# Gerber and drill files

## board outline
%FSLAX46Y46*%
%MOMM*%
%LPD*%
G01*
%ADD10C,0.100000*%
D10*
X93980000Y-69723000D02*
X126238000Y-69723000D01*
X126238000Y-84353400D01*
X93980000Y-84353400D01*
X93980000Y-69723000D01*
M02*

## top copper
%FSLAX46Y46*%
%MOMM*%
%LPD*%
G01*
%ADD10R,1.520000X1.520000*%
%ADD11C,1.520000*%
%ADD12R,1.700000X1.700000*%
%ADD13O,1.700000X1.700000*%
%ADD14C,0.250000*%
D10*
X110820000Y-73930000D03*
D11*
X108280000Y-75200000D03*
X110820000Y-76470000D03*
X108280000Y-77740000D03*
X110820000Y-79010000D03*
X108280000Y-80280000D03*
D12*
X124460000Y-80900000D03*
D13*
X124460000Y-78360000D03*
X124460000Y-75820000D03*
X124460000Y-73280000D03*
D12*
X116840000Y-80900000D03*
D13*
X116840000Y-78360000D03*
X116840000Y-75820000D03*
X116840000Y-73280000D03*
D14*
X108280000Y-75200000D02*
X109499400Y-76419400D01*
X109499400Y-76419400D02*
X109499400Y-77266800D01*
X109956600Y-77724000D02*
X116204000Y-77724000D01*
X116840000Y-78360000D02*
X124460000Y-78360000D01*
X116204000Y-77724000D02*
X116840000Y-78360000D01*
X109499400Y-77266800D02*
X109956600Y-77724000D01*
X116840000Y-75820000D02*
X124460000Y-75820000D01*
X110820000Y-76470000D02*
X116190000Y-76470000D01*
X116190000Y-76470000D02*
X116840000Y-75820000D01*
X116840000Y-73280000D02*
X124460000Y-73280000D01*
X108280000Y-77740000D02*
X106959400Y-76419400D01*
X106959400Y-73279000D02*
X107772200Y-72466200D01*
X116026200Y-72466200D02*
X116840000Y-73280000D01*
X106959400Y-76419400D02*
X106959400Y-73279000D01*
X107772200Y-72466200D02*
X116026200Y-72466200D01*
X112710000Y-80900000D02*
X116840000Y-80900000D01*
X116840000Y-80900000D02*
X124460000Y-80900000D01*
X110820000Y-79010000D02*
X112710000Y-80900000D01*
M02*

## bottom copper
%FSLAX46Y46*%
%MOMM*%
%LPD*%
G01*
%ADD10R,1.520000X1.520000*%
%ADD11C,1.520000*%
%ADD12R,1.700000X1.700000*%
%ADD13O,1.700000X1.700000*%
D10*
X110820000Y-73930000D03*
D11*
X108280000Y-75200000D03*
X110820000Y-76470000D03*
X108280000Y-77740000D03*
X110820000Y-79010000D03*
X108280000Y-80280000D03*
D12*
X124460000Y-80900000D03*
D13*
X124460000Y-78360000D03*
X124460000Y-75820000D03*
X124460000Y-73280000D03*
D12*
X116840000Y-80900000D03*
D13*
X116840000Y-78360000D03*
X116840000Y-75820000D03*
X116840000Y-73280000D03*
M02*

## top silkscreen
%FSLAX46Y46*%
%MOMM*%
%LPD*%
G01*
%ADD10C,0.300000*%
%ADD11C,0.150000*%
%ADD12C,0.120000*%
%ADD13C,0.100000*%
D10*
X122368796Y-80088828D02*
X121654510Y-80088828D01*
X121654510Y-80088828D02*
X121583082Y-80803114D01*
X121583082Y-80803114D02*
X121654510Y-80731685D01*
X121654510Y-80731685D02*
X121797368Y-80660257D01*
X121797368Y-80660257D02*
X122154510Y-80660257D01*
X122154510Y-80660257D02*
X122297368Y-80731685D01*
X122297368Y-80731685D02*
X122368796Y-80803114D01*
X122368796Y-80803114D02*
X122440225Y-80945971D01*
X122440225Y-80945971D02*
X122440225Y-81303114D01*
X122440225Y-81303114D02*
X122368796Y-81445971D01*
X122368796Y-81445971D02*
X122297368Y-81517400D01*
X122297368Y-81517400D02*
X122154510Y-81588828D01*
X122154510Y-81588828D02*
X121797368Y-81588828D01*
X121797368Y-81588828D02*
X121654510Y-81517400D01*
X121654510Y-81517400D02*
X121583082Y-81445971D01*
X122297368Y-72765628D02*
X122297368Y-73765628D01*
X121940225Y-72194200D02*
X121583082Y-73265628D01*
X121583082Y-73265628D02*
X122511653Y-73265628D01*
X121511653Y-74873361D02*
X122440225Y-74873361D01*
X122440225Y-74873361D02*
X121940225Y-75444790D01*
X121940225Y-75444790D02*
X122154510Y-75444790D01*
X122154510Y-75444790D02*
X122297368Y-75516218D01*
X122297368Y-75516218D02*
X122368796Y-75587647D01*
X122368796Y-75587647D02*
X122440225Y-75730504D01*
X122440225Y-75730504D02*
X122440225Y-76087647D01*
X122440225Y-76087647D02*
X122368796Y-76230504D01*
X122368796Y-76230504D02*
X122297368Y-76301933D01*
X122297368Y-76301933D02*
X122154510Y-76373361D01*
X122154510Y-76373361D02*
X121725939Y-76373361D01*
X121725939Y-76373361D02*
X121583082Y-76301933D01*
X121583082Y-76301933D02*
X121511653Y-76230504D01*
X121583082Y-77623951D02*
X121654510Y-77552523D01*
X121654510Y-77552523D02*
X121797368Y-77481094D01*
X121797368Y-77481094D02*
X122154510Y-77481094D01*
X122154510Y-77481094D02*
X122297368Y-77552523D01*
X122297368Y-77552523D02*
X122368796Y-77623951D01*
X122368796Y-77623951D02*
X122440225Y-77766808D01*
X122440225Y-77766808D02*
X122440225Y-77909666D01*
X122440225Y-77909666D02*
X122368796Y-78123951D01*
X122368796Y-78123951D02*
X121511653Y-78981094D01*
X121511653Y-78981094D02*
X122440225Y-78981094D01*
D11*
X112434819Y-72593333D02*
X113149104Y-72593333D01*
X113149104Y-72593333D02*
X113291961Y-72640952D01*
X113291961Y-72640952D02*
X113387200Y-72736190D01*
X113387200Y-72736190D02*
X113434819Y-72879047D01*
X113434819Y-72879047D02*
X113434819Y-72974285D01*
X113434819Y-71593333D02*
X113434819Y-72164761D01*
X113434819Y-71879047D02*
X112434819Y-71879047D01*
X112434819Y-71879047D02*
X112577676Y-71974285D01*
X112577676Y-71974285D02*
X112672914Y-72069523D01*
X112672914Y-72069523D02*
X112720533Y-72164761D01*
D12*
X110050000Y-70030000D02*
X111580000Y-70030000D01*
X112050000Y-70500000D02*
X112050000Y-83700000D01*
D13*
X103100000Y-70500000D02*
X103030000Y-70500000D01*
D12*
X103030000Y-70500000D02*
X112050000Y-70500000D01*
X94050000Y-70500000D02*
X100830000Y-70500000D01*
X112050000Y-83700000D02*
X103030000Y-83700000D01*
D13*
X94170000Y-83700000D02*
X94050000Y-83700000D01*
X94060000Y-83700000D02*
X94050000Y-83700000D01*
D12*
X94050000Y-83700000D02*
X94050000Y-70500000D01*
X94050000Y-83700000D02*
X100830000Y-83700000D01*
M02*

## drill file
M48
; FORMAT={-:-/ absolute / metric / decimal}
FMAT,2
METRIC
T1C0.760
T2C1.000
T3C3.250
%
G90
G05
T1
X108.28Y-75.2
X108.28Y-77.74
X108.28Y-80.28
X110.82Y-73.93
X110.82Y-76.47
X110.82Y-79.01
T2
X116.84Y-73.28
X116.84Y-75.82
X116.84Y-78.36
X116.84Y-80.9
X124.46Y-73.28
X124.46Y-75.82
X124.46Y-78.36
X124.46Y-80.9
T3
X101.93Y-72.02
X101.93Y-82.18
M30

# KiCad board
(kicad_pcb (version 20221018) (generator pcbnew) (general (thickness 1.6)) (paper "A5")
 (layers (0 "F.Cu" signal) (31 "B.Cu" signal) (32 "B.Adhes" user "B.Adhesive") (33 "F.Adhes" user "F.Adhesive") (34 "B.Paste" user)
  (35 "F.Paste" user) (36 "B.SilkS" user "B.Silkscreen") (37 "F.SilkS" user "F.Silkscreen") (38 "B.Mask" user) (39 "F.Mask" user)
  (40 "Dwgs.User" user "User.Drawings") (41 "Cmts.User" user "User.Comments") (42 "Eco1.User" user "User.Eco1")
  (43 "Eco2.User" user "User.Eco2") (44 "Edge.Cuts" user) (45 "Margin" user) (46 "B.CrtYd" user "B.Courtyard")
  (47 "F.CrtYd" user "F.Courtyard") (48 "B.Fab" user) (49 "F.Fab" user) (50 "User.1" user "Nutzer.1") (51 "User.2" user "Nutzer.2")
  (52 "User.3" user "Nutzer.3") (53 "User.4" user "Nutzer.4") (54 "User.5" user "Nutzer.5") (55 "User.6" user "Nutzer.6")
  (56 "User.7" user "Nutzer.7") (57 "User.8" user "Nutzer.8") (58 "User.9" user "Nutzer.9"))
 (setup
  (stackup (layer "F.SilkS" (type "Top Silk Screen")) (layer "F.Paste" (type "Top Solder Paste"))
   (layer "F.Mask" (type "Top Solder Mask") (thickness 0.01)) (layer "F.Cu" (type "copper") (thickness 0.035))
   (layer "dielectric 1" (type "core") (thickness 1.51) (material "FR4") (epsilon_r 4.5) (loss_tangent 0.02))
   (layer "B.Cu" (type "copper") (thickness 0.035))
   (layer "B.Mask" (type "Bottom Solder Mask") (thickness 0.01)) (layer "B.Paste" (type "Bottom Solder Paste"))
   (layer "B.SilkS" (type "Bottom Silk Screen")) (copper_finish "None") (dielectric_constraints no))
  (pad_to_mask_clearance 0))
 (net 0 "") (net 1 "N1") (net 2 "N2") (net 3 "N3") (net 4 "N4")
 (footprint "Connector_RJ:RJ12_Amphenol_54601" (layer "F.Cu") (at 110.82 73.93 -90)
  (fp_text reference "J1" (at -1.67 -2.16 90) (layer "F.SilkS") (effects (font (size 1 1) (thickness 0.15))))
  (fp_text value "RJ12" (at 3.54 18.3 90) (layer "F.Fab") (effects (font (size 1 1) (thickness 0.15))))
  (fp_line (start -3.9 0.77) (end -3.9 -0.76) (stroke (width 0.12) (type solid)) (layer "F.SilkS"))
  (fp_line (start -3.43 -1.23) (end 9.77 -1.23) (stroke (width 0.12) (type solid)) (layer "F.SilkS"))
  (fp_line (start -3.43 7.72) (end -3.43 7.79) (stroke (width 0.1) (type solid)) (layer "F.SilkS"))
  (fp_line (start -3.43 7.79) (end -3.43 -1.23) (stroke (width 0.12) (type solid)) (layer "F.SilkS"))
  (fp_line (start -3.43 16.77) (end -3.43 9.99) (stroke (width 0.12) (type solid)) (layer "F.SilkS"))
  (fp_line (start 9.77 -1.23) (end 9.77 7.79) (stroke (width 0.12) (type solid)) (layer "F.SilkS"))
  (fp_line (start 9.77 16.65) (end 9.77 16.77) (stroke (width 0.1) (type solid)) (layer "F.SilkS"))
  (fp_line (start 9.77 16.76) (end 9.77 16.77) (stroke (width 0.1) (type solid)) (layer "F.SilkS"))
  (fp_line (start 9.77 16.77) (end -3.43 16.77) (stroke (width 0.12) (type solid)) (layer "F.SilkS"))
  (fp_line (start 9.77 16.77) (end 9.77 9.99) (stroke (width 0.12) (type solid)) (layer "F.SilkS"))
  (pad "" np_thru_hole circle (at -1.91 8.89 270) (size 3.25 3.25) (drill 3.25) (layers "*.Cu" "*.Mask"))
  (pad "" np_thru_hole circle (at 8.25 8.89 270) (size 3.25 3.25) (drill 3.25) (layers "*.Cu" "*.Mask"))
  (pad "1" thru_hole rect (at 0 0 270) (size 1.52 1.52) (drill 0.76) (layers "*.Cu" "*.Mask"))
  (pad "2" thru_hole circle (at 1.27 2.54 270) (size 1.52 1.52) (drill 0.76) (layers "*.Cu" "*.Mask") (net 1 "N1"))
  (pad "3" thru_hole circle (at 2.54 0 270) (size 1.52 1.52) (drill 0.76) (layers "*.Cu" "*.Mask") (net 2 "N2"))
  (pad "4" thru_hole circle (at 3.81 2.54 270) (size 1.52 1.52) (drill 0.76) (layers "*.Cu" "*.Mask") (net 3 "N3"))
  (pad "5" thru_hole circle (at 5.08 0 270) (size 1.52 1.52) (drill 0.76) (layers "*.Cu" "*.Mask") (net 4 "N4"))
  (pad "6" thru_hole circle (at 6.35 2.54 270) (size 1.52 1.52) (drill 0.76) (layers "*.Cu" "*.Mask")))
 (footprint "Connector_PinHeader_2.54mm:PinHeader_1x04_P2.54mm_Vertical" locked (layer "B.Cu") (at 124.46 80.9)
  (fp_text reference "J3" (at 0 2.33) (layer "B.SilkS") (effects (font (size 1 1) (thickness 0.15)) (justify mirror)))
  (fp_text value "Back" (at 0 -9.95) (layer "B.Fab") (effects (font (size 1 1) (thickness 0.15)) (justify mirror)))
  (pad "1" thru_hole rect locked (at 0 0) (size 1.7 1.7) (drill 1) (layers "*.Cu" "*.Mask") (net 4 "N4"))
  (pad "2" thru_hole oval locked (at 0 -2.54) (size 1.7 1.7) (drill 1) (layers "*.Cu" "*.Mask") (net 1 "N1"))
  (pad "3" thru_hole oval locked (at 0 -5.08) (size 1.7 1.7) (drill 1) (layers "*.Cu" "*.Mask") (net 2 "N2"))
  (pad "4" thru_hole oval locked (at 0 -7.62) (size 1.7 1.7) (drill 1) (layers "*.Cu" "*.Mask") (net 3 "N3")))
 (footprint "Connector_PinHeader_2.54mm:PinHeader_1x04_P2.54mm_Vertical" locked (layer "B.Cu") (at 116.84 80.9)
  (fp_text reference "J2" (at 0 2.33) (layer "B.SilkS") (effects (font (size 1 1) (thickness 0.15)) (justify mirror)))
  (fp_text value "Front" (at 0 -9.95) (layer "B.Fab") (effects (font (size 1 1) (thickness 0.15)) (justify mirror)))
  (pad "1" thru_hole rect locked (at 0 0) (size 1.7 1.7) (drill 1) (layers "*.Cu" "*.Mask") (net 4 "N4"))
  (pad "2" thru_hole oval locked (at 0 -2.54) (size 1.7 1.7) (drill 1) (layers "*.Cu" "*.Mask") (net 1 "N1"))
  (pad "3" thru_hole oval locked (at 0 -5.08) (size 1.7 1.7) (drill 1) (layers "*.Cu" "*.Mask") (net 2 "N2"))
  (pad "4" thru_hole oval locked (at 0 -7.62) (size 1.7 1.7) (drill 1) (layers "*.Cu" "*.Mask") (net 3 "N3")))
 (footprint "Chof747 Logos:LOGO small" (layer "B.Cu") (at 97.5614 77.3684 180)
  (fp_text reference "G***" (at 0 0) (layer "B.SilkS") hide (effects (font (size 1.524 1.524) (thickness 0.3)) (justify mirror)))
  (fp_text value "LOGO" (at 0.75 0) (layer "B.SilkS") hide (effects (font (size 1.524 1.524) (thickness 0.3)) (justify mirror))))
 (gr_rect (start 93.98 69.723) (end 126.238 84.3534) (stroke (width 0.1) (type default)) (fill none) (layer "Edge.Cuts"))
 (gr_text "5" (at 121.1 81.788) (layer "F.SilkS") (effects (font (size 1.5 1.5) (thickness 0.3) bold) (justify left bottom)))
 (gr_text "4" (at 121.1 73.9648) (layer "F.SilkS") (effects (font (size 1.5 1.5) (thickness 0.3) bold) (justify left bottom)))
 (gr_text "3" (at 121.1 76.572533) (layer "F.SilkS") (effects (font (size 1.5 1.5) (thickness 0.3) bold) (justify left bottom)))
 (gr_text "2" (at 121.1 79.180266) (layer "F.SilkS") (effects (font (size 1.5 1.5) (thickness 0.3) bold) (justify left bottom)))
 (segment (start 108.28 75.2) (end 109.4994 76.4194) (width 0.25) (layer "F.Cu") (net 1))
 (segment (start 109.4994 76.4194) (end 109.4994 77.2668) (width 0.25) (layer "F.Cu") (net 1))
 (segment (start 109.9566 77.724) (end 116.204 77.724) (width 0.25) (layer "F.Cu") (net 1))
 (segment (start 116.84 78.36) (end 124.46 78.36) (width 0.25) (layer "F.Cu") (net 1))
 (segment (start 116.204 77.724) (end 116.84 78.36) (width 0.25) (layer "F.Cu") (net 1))
 (segment (start 109.4994 77.2668) (end 109.9566 77.724) (width 0.25) (layer "F.Cu") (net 1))
 (segment (start 116.84 75.82) (end 124.46 75.82) (width 0.25) (layer "F.Cu") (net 2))
 (segment (start 110.82 76.47) (end 116.19 76.47) (width 0.25) (layer "F.Cu") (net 2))
 (segment (start 116.19 76.47) (end 116.84 75.82) (width 0.25) (layer "F.Cu") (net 2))
 (segment (start 116.84 73.28) (end 124.46 73.28) (width 0.25) (layer "F.Cu") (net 3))
 (segment (start 108.28 77.74) (end 106.9594 76.4194) (width 0.25) (layer "F.Cu") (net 3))
 (segment (start 106.9594 73.279) (end 107.7722 72.4662) (width 0.25) (layer "F.Cu") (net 3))
 (segment (start 116.0262 72.4662) (end 116.84 73.28) (width 0.25) (layer "F.Cu") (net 3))
 (segment (start 106.9594 76.4194) (end 106.9594 73.279) (width 0.25) (layer "F.Cu") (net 3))
 (segment (start 107.7722 72.4662) (end 116.0262 72.4662) (width 0.25) (layer "F.Cu") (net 3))
 (segment (start 112.71 80.9) (end 116.84 80.9) (width 0.25) (layer "F.Cu") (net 4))
 (segment (start 116.84 80.9) (end 124.46 80.9) (width 0.25) (layer "F.Cu") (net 4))
 (segment (start 110.82 79.01) (end 112.71 80.9) (width 0.25) (layer "F.Cu") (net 4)))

